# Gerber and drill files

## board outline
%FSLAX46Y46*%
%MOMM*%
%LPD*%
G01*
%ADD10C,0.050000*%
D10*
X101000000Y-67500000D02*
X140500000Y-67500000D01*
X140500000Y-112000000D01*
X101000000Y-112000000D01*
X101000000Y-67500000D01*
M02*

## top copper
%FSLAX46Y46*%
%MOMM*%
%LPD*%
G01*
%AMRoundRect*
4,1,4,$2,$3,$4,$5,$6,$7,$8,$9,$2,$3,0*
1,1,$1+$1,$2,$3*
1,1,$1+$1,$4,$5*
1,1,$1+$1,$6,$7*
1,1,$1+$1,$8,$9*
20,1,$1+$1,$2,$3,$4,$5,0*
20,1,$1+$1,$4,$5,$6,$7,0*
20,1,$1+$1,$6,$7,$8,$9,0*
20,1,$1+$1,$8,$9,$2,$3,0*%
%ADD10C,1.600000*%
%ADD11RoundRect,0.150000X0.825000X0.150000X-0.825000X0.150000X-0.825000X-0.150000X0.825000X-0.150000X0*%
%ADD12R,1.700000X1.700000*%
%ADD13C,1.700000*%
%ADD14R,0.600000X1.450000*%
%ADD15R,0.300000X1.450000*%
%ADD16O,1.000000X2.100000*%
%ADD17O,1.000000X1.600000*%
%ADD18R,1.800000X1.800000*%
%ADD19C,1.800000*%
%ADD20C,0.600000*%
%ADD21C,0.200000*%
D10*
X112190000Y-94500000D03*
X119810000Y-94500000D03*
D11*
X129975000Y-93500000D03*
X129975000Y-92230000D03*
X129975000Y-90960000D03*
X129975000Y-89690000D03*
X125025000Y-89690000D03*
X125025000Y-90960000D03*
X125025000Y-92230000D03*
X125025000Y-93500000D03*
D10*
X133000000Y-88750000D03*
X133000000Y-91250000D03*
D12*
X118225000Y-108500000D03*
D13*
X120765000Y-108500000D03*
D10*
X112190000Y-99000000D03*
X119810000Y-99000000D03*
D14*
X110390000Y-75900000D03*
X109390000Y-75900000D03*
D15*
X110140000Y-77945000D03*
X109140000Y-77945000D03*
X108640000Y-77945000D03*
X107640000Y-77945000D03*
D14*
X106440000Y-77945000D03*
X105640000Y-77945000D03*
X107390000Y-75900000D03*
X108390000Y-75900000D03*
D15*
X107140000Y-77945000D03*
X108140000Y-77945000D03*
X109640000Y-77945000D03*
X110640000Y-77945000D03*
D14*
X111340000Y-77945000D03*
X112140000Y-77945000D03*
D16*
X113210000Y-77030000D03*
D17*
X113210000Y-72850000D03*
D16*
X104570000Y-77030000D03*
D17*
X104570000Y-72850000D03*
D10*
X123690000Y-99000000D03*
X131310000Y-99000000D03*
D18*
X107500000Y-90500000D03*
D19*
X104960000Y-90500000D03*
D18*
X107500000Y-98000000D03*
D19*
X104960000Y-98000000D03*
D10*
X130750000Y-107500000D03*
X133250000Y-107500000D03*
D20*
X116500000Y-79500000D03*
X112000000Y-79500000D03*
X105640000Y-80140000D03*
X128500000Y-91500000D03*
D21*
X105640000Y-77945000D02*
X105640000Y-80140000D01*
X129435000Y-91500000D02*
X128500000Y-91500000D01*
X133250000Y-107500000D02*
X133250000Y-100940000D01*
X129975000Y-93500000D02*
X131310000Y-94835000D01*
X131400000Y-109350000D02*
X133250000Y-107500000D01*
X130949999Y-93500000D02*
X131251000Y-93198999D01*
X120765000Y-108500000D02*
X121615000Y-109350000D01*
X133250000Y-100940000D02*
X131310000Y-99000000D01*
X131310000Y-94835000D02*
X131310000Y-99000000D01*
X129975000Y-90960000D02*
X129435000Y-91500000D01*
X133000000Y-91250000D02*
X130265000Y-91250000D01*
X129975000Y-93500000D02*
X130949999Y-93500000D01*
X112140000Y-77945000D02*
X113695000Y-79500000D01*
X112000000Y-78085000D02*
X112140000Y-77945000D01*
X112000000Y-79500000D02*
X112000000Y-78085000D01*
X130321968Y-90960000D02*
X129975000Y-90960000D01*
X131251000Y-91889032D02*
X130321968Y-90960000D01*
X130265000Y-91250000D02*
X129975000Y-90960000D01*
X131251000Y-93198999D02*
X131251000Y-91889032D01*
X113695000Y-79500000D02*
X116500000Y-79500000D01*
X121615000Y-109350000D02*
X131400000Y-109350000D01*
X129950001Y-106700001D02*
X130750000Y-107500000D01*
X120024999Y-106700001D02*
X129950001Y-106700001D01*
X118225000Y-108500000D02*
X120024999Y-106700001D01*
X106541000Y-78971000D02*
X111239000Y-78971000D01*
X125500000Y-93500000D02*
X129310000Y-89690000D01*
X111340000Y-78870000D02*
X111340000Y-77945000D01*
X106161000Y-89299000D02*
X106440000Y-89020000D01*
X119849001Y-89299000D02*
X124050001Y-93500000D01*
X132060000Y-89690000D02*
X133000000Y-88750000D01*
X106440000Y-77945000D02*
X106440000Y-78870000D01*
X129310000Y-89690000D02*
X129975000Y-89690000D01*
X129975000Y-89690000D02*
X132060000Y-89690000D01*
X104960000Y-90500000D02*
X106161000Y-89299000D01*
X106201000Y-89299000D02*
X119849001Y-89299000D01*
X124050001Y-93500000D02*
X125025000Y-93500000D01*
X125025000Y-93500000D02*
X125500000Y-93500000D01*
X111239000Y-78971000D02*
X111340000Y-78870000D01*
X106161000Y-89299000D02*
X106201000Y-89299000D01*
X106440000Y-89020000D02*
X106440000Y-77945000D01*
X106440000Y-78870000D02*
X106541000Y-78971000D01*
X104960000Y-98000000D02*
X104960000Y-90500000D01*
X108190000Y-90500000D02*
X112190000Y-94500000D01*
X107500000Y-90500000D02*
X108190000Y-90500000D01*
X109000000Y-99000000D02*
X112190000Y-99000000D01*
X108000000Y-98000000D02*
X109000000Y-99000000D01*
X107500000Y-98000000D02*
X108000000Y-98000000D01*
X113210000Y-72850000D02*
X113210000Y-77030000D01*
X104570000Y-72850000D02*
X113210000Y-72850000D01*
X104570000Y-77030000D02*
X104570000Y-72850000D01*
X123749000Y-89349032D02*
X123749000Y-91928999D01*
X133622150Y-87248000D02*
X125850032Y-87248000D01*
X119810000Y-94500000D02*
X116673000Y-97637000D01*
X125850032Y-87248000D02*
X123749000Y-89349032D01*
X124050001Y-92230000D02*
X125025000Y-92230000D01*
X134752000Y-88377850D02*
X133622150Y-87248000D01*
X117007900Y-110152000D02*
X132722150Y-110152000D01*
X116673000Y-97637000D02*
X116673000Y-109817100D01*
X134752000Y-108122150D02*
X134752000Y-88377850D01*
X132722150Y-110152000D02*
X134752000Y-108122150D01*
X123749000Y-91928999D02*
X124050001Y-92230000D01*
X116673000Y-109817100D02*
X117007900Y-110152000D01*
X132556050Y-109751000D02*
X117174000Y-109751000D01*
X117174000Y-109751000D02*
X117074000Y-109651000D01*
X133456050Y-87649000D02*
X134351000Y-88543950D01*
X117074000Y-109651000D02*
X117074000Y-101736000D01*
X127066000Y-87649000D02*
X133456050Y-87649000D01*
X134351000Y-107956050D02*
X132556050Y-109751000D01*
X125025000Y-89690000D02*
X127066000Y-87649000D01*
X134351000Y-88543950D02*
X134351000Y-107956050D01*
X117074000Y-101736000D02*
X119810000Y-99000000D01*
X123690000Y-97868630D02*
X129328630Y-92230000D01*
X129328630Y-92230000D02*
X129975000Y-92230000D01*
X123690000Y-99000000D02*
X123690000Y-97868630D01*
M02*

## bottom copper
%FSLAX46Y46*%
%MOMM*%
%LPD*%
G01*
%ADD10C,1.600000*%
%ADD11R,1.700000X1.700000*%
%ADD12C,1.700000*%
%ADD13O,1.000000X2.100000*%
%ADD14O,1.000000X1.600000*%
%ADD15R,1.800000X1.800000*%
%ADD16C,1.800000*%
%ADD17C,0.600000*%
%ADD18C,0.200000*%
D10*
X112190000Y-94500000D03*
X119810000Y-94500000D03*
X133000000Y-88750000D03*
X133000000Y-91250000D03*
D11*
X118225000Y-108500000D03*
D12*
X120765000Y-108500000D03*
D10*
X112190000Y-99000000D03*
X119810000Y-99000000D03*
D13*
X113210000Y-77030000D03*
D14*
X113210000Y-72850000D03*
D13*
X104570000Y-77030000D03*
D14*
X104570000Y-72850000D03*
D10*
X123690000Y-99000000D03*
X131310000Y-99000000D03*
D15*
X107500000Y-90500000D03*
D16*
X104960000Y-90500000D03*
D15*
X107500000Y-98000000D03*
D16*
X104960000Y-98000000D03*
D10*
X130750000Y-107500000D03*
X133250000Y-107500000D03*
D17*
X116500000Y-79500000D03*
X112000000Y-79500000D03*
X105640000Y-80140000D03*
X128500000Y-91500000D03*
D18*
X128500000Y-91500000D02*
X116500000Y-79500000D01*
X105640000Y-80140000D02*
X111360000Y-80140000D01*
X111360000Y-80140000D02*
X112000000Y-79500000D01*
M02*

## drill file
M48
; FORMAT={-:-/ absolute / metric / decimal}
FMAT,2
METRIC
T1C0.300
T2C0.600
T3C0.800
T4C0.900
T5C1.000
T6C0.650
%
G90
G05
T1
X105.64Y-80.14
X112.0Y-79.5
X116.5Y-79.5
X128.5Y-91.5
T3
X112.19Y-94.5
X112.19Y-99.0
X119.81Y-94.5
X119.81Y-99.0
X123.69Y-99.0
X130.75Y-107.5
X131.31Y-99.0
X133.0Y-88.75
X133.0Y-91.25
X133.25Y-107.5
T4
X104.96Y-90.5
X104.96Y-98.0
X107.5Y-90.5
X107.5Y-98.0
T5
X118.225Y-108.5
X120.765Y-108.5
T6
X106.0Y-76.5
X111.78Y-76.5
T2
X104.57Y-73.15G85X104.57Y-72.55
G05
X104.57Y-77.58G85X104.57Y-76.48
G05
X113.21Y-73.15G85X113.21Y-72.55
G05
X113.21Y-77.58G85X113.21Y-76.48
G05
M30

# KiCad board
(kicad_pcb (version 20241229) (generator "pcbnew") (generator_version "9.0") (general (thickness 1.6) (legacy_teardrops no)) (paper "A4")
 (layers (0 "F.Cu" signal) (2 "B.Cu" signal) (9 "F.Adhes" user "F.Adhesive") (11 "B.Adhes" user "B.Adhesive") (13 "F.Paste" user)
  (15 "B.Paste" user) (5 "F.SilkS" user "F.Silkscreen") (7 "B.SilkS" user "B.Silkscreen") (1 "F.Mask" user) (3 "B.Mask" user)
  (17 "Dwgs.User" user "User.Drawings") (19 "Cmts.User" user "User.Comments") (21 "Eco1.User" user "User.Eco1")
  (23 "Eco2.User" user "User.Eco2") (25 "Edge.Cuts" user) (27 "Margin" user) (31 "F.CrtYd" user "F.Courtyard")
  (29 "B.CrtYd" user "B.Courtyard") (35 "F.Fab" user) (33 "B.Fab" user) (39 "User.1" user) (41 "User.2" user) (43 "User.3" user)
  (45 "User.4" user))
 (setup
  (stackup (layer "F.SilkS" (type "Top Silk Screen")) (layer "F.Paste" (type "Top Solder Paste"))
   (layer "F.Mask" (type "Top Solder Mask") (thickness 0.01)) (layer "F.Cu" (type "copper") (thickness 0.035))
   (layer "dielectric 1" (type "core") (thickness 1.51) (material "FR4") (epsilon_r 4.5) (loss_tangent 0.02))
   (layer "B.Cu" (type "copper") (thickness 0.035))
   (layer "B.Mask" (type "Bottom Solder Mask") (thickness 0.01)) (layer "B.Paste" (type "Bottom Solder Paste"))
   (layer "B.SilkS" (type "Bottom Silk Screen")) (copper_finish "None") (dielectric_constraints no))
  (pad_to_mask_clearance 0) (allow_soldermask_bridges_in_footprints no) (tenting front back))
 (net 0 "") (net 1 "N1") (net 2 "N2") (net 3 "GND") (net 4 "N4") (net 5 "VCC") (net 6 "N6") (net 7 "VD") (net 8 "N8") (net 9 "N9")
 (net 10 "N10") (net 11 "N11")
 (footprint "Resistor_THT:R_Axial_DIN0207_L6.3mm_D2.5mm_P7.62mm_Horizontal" (layer "F.Cu") (at 112.19 94.5)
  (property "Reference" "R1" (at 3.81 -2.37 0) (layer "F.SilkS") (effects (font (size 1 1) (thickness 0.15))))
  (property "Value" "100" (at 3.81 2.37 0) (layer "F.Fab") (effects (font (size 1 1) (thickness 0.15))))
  (pad "1" thru_hole circle (at 0 0) (size 1.6 1.6) (drill 0.8) (layers "*.Cu" "*.Mask") (remove_unused_layers no) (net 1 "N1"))
  (pad "2" thru_hole circle (at 7.62 0) (size 1.6 1.6) (drill 0.8) (layers "*.Cu" "*.Mask") (remove_unused_layers no) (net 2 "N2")))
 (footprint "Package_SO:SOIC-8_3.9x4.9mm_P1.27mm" (layer "F.Cu") (at 127.5 91.595 180)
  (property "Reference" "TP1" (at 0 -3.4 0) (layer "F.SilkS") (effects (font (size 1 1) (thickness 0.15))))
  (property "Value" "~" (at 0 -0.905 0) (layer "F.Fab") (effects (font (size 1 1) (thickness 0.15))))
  (pad "1" smd roundrect (at -2.475 -1.905 180) (size 1.95 0.6) (layers "F.Cu" "F.Mask" "F.Paste") (roundrect_rratio 0.25) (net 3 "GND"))
  (pad "2" smd roundrect (at -2.475 -0.635 180) (size 1.95 0.6) (layers "F.Cu" "F.Mask" "F.Paste") (roundrect_rratio 0.25) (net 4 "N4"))
  (pad "3" smd roundrect (at -2.475 0.635 180) (size 1.95 0.6) (layers "F.Cu" "F.Mask" "F.Paste") (roundrect_rratio 0.25) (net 3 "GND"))
  (pad "4" smd roundrect (at -2.475 1.905 180) (size 1.95 0.6) (layers "F.Cu" "F.Mask" "F.Paste") (roundrect_rratio 0.25) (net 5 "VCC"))
  (pad "5" smd roundrect (at 2.475 1.905 180) (size 1.95 0.6) (layers "F.Cu" "F.Mask" "F.Paste") (roundrect_rratio 0.25) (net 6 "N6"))
  (pad "6" smd roundrect (at 2.475 0.635 180) (size 1.95 0.6) (layers "F.Cu" "F.Mask" "F.Paste") (roundrect_rratio 0.25))
  (pad "7" smd roundrect (at 2.475 -0.635 180) (size 1.95 0.6) (layers "F.Cu" "F.Mask" "F.Paste") (roundrect_rratio 0.25) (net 2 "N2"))
  (pad "8" smd roundrect (at 2.475 -1.905 180) (size 1.95 0.6) (layers "F.Cu" "F.Mask" "F.Paste") (roundrect_rratio 0.25) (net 5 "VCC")))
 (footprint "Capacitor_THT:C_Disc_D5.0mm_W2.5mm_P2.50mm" (layer "F.Cu") (at 133 88.75 -90)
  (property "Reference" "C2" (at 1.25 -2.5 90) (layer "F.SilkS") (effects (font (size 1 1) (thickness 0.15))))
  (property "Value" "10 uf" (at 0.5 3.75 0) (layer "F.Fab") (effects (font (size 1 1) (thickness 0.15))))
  (pad "1" thru_hole circle (at 0 0 270) (size 1.6 1.6) (drill 0.8) (layers "*.Cu" "*.Mask") (remove_unused_layers no) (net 5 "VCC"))
  (pad "2" thru_hole circle (at 2.5 0 270) (size 1.6 1.6) (drill 0.8) (layers "*.Cu" "*.Mask") (remove_unused_layers no) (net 3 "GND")))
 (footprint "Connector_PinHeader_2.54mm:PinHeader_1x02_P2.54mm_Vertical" (layer "F.Cu") (at 118.225 108.5 90)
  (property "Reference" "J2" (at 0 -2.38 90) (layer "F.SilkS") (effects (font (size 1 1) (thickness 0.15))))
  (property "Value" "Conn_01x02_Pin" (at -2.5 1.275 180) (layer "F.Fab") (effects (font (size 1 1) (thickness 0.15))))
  (pad "1" thru_hole rect (at 0 0 90) (size 1.7 1.7) (drill 1) (layers "*.Cu" "*.Mask") (remove_unused_layers no) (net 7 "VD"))
  (pad "2" thru_hole circle (at 0 2.54 90) (size 1.7 1.7) (drill 1) (layers "*.Cu" "*.Mask") (remove_unused_layers no) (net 3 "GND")))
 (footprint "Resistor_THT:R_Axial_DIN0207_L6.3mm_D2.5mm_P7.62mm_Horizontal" (layer "F.Cu") (at 112.19 99)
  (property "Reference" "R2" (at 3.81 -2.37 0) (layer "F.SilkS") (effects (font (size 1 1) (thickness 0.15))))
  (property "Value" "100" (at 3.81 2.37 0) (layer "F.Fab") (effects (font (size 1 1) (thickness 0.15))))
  (pad "1" thru_hole circle (at 0 0) (size 1.6 1.6) (drill 0.8) (layers "*.Cu" "*.Mask") (remove_unused_layers no) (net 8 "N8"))
  (pad "2" thru_hole circle (at 7.62 0) (size 1.6 1.6) (drill 0.8) (layers "*.Cu" "*.Mask") (remove_unused_layers no) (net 6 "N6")))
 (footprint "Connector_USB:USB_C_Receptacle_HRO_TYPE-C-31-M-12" (layer "F.Cu") (at 108.89 73.9 180)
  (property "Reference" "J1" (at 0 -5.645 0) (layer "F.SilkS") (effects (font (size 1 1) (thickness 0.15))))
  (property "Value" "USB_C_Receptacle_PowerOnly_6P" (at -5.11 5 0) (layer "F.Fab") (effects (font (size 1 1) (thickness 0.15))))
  (pad "" np_thru_hole circle (at -2.89 -2.6 180) (size 0.65 0.65) (drill 0.65) (layers "*.Cu" "*.Mask"))
  (pad "" np_thru_hole circle (at 2.89 -2.6 180) (size 0.65 0.65) (drill 0.65) (layers "*.Cu" "*.Mask"))
  (pad "A1" smd rect (at -1.5 -2 180) (size 0.6 1.45) (layers "F.Cu" "F.Mask" "F.Paste"))
  (pad "A4" smd rect (at -0.5 -2 180) (size 0.6 1.45) (layers "F.Cu" "F.Mask" "F.Paste"))
  (pad "A5" smd rect (at -1.25 -4.045 180) (size 0.3 1.45) (layers "F.Cu" "F.Mask" "F.Paste") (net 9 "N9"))
  (pad "A6" smd rect (at -0.25 -4.045 180) (size 0.3 1.45) (layers "F.Cu" "F.Mask" "F.Paste"))
  (pad "A7" smd rect (at 0.25 -4.045 180) (size 0.3 1.45) (layers "F.Cu" "F.Mask" "F.Paste"))
  (pad "A8" smd rect (at 1.25 -4.045 180) (size 0.3 1.45) (layers "F.Cu" "F.Mask" "F.Paste"))
  (pad "A9" smd rect (at 2.45 -4.045 180) (size 0.6 1.45) (layers "F.Cu" "F.Mask" "F.Paste") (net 5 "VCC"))
  (pad "A12" smd rect (at 3.25 -4.045 180) (size 0.6 1.45) (layers "F.Cu" "F.Mask" "F.Paste") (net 3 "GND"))
  (pad "B1" smd rect (at 1.5 -2 180) (size 0.6 1.45) (layers "F.Cu" "F.Mask" "F.Paste"))
  (pad "B4" smd rect (at 0.5 -2 180) (size 0.6 1.45) (layers "F.Cu" "F.Mask" "F.Paste"))
  (pad "B5" smd rect (at 1.75 -4.045 180) (size 0.3 1.45) (layers "F.Cu" "F.Mask" "F.Paste") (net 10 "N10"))
  (pad "B6" smd rect (at 0.75 -4.045 180) (size 0.3 1.45) (layers "F.Cu" "F.Mask" "F.Paste"))
  (pad "B7" smd rect (at -0.75 -4.045 180) (size 0.3 1.45) (layers "F.Cu" "F.Mask" "F.Paste"))
  (pad "B8" smd rect (at -1.75 -4.045 180) (size 0.3 1.45) (layers "F.Cu" "F.Mask" "F.Paste"))
  (pad "B9" smd rect (at -2.45 -4.045 180) (size 0.6 1.45) (layers "F.Cu" "F.Mask" "F.Paste") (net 5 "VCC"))
  (pad "B12" smd rect (at -3.25 -4.045 180) (size 0.6 1.45) (layers "F.Cu" "F.Mask" "F.Paste") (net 3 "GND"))
  (pad "S1" thru_hole oval (at -4.32 -3.13 180) (size 1 2.1) (drill oval 0.6 1.7) (layers "*.Cu" "*.Mask") (remove_unused_layers no)
   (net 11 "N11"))
  (pad "S1" thru_hole oval (at -4.32 1.05 180) (size 1 1.6) (drill oval 0.6 1.2) (layers "*.Cu" "*.Mask") (remove_unused_layers no)
   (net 11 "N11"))
  (pad "S1" thru_hole oval (at 4.32 -3.13 180) (size 1 2.1) (drill oval 0.6 1.7) (layers "*.Cu" "*.Mask") (remove_unused_layers no)
   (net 11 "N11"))
  (pad "S1" thru_hole oval (at 4.32 1.05 180) (size 1 1.6) (drill oval 0.6 1.2) (layers "*.Cu" "*.Mask") (remove_unused_layers no)
   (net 11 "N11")))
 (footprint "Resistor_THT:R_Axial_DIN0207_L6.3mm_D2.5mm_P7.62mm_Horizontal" (layer "F.Cu") (at 123.69 99)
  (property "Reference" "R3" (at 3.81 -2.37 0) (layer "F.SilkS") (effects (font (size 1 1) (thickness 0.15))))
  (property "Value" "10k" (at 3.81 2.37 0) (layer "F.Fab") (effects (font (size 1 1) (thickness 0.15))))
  (pad "1" thru_hole circle (at 0 0) (size 1.6 1.6) (drill 0.8) (layers "*.Cu" "*.Mask") (remove_unused_layers no) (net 4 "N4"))
  (pad "2" thru_hole circle (at 7.62 0) (size 1.6 1.6) (drill 0.8) (layers "*.Cu" "*.Mask") (remove_unused_layers no) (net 3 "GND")))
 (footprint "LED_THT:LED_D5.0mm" (layer "F.Cu") (at 107.5 90.5 180)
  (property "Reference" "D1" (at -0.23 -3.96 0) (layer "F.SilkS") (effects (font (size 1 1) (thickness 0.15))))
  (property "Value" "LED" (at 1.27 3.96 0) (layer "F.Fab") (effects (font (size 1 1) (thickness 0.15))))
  (pad "1" thru_hole rect (at 0 0 180) (size 1.8 1.8) (drill 0.9) (layers "*.Cu" "*.Mask") (remove_unused_layers no) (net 1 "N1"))
  (pad "2" thru_hole circle (at 2.54 0 180) (size 1.8 1.8) (drill 0.9) (layers "*.Cu" "*.Mask") (remove_unused_layers no) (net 5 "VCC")))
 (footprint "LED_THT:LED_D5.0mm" (layer "F.Cu") (at 107.5 98 180)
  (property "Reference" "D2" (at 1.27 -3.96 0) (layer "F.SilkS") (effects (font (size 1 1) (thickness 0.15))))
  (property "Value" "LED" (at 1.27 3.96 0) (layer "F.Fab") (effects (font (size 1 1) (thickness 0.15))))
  (pad "1" thru_hole rect (at 0 0 180) (size 1.8 1.8) (drill 0.9) (layers "*.Cu" "*.Mask") (remove_unused_layers no) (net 8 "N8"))
  (pad "2" thru_hole circle (at 2.54 0 180) (size 1.8 1.8) (drill 0.9) (layers "*.Cu" "*.Mask") (remove_unused_layers no) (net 5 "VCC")))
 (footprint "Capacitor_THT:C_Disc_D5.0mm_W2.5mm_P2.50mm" (layer "F.Cu") (at 130.75 107.5)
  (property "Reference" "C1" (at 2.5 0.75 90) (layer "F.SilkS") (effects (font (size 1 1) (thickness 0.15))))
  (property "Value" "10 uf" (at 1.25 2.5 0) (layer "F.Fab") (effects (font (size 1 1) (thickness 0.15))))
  (pad "1" thru_hole circle (at 0 0) (size 1.6 1.6) (drill 0.8) (layers "*.Cu" "*.Mask") (remove_unused_layers no) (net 7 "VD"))
  (pad "2" thru_hole circle (at 2.5 0) (size 1.6 1.6) (drill 0.8) (layers "*.Cu" "*.Mask") (remove_unused_layers no) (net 3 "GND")))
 (gr_rect (start 101 67.5) (end 140.5 112) (stroke (width 0.05) (type default)) (fill no) (layer "Edge.Cuts"))
 (segment (start 105.64 77.945) (end 105.64 80.14) (width 0.2) (layer "F.Cu") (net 3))
 (segment (start 129.435 91.5) (end 128.5 91.5) (width 0.2) (layer "F.Cu") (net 3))
 (segment (start 133.25 107.5) (end 133.25 100.94) (width 0.2) (layer "F.Cu") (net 3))
 (segment (start 129.975 93.5) (end 131.31 94.835) (width 0.2) (layer "F.Cu") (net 3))
 (segment (start 131.4 109.35) (end 133.25 107.5) (width 0.2) (layer "F.Cu") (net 3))
 (segment (start 130.949999 93.5) (end 131.251 93.198999) (width 0.2) (layer "F.Cu") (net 3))
 (segment (start 120.765 108.5) (end 121.615 109.35) (width 0.2) (layer "F.Cu") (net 3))
 (segment (start 133.25 100.94) (end 131.31 99) (width 0.2) (layer "F.Cu") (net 3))
 (segment (start 131.31 94.835) (end 131.31 99) (width 0.2) (layer "F.Cu") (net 3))
 (segment (start 129.975 90.96) (end 129.435 91.5) (width 0.2) (layer "F.Cu") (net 3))
 (segment (start 133 91.25) (end 130.265 91.25) (width 0.2) (layer "F.Cu") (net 3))
 (segment (start 129.975 93.5) (end 130.949999 93.5) (width 0.2) (layer "F.Cu") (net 3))
 (segment (start 112.14 77.945) (end 113.695 79.5) (width 0.2) (layer "F.Cu") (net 3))
 (segment (start 112 78.085) (end 112.14 77.945) (width 0.2) (layer "F.Cu") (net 3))
 (segment (start 112 79.5) (end 112 78.085) (width 0.2) (layer "F.Cu") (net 3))
 (segment (start 130.321968 90.96) (end 129.975 90.96) (width 0.2) (layer "F.Cu") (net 3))
 (segment (start 131.251 91.889032) (end 130.321968 90.96) (width 0.2) (layer "F.Cu") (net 3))
 (segment (start 130.265 91.25) (end 129.975 90.96) (width 0.2) (layer "F.Cu") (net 3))
 (segment (start 131.251 93.198999) (end 131.251 91.889032) (width 0.2) (layer "F.Cu") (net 3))
 (segment (start 113.695 79.5) (end 116.5 79.5) (width 0.2) (layer "F.Cu") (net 3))
 (segment (start 121.615 109.35) (end 131.4 109.35) (width 0.2) (layer "F.Cu") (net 3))
 (via (at 116.5 79.5) (size 0.6) (drill 0.3) (layers "F.Cu" "B.Cu") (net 3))
 (via (at 112 79.5) (size 0.6) (drill 0.3) (layers "F.Cu" "B.Cu") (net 3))
 (via (at 105.64 80.14) (size 0.6) (drill 0.3) (layers "F.Cu" "B.Cu") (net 3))
 (via (at 128.5 91.5) (size 0.6) (drill 0.3) (layers "F.Cu" "B.Cu") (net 3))
 (segment (start 128.5 91.5) (end 116.5 79.5) (width 0.2) (layer "B.Cu") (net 3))
 (segment (start 105.64 80.14) (end 111.36 80.14) (width 0.2) (layer "B.Cu") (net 3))
 (segment (start 111.36 80.14) (end 112 79.5) (width 0.2) (layer "B.Cu") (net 3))
 (segment (start 129.950001 106.700001) (end 130.75 107.5) (width 0.2) (layer "F.Cu") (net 7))
 (segment (start 120.024999 106.700001) (end 129.950001 106.700001) (width 0.2) (layer "F.Cu") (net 7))
 (segment (start 118.225 108.5) (end 120.024999 106.700001) (width 0.2) (layer "F.Cu") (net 7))
 (segment (start 106.541 78.971) (end 111.239 78.971) (width 0.2) (layer "F.Cu") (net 5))
 (segment (start 125.5 93.5) (end 129.31 89.69) (width 0.2) (layer "F.Cu") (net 5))
 (segment (start 111.34 78.87) (end 111.34 77.945) (width 0.2) (layer "F.Cu") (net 5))
 (segment (start 106.161 89.299) (end 106.44 89.02) (width 0.2) (layer "F.Cu") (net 5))
 (segment (start 119.849001 89.299) (end 124.050001 93.5) (width 0.2) (layer "F.Cu") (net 5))
 (segment (start 132.06 89.69) (end 133 88.75) (width 0.2) (layer "F.Cu") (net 5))
 (segment (start 106.44 77.945) (end 106.44 78.87) (width 0.2) (layer "F.Cu") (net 5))
 (segment (start 129.31 89.69) (end 129.975 89.69) (width 0.2) (layer "F.Cu") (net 5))
 (segment (start 129.975 89.69) (end 132.06 89.69) (width 0.2) (layer "F.Cu") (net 5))
 (segment (start 104.96 90.5) (end 106.161 89.299) (width 0.2) (layer "F.Cu") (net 5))
 (segment (start 106.201 89.299) (end 119.849001 89.299) (width 0.2) (layer "F.Cu") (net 5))
 (segment (start 124.050001 93.5) (end 125.025 93.5) (width 0.2) (layer "F.Cu") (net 5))
 (segment (start 125.025 93.5) (end 125.5 93.5) (width 0.2) (layer "F.Cu") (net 5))
 (segment (start 111.239 78.971) (end 111.34 78.87) (width 0.2) (layer "F.Cu") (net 5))
 (segment (start 106.161 89.299) (end 106.201 89.299) (width 0.2) (layer "F.Cu") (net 5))
 (segment (start 106.44 89.02) (end 106.44 77.945) (width 0.2) (layer "F.Cu") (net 5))
 (segment (start 106.44 78.87) (end 106.541 78.971) (width 0.2) (layer "F.Cu") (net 5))
 (segment (start 104.96 98) (end 104.96 90.5) (width 0.2) (layer "F.Cu") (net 5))
 (segment (start 108.19 90.5) (end 112.19 94.5) (width 0.2) (layer "F.Cu") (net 1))
 (segment (start 107.5 90.5) (end 108.19 90.5) (width 0.2) (layer "F.Cu") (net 1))
 (segment (start 109 99) (end 112.19 99) (width 0.2) (layer "F.Cu") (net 8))
 (segment (start 108 98) (end 109 99) (width 0.2) (layer "F.Cu") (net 8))
 (segment (start 107.5 98) (end 108 98) (width 0.2) (layer "F.Cu") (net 8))
 (segment (start 113.21 72.85) (end 113.21 77.03) (width 0.2) (layer "F.Cu") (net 11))
 (segment (start 104.57 72.85) (end 113.21 72.85) (width 0.2) (layer "F.Cu") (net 11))
 (segment (start 104.57 77.03) (end 104.57 72.85) (width 0.2) (layer "F.Cu") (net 11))
 (segment (start 123.749 89.349032) (end 123.749 91.928999) (width 0.2) (layer "F.Cu") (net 2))
 (segment (start 133.62215 87.248) (end 125.850032 87.248) (width 0.2) (layer "F.Cu") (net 2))
 (segment (start 119.81 94.5) (end 116.673 97.637) (width 0.2) (layer "F.Cu") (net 2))
 (segment (start 125.850032 87.248) (end 123.749 89.349032) (width 0.2) (layer "F.Cu") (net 2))
 (segment (start 124.050001 92.23) (end 125.025 92.23) (width 0.2) (layer "F.Cu") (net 2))
 (segment (start 134.752 88.37785) (end 133.62215 87.248) (width 0.2) (layer "F.Cu") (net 2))
 (segment (start 117.0079 110.152) (end 132.72215 110.152) (width 0.2) (layer "F.Cu") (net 2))
 (segment (start 116.673 97.637) (end 116.673 109.8171) (width 0.2) (layer "F.Cu") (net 2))
 (segment (start 134.752 108.12215) (end 134.752 88.37785) (width 0.2) (layer "F.Cu") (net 2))
 (segment (start 132.72215 110.152) (end 134.752 108.12215) (width 0.2) (layer "F.Cu") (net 2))
 (segment (start 123.749 91.928999) (end 124.050001 92.23) (width 0.2) (layer "F.Cu") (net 2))
 (segment (start 116.673 109.8171) (end 117.0079 110.152) (width 0.2) (layer "F.Cu") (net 2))
 (segment (start 132.55605 109.751) (end 117.174 109.751) (width 0.2) (layer "F.Cu") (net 6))
 (segment (start 117.174 109.751) (end 117.074 109.651) (width 0.2) (layer "F.Cu") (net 6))
 (segment (start 133.45605 87.649) (end 134.351 88.54395) (width 0.2) (layer "F.Cu") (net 6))
 (segment (start 117.074 109.651) (end 117.074 101.736) (width 0.2) (layer "F.Cu") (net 6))
 (segment (start 127.066 87.649) (end 133.45605 87.649) (width 0.2) (layer "F.Cu") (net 6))
 (segment (start 134.351 107.95605) (end 132.55605 109.751) (width 0.2) (layer "F.Cu") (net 6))
 (segment (start 125.025 89.69) (end 127.066 87.649) (width 0.2) (layer "F.Cu") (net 6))
 (segment (start 134.351 88.54395) (end 134.351 107.95605) (width 0.2) (layer "F.Cu") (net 6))
 (segment (start 117.074 101.736) (end 119.81 99) (width 0.2) (layer "F.Cu") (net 6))
 (segment (start 123.69 97.86863) (end 129.32863 92.23) (width 0.2) (layer "F.Cu") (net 4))
 (segment (start 129.32863 92.23) (end 129.975 92.23) (width 0.2) (layer "F.Cu") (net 4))
 (segment (start 123.69 99) (end 123.69 97.86863) (width 0.2) (layer "F.Cu") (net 4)))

